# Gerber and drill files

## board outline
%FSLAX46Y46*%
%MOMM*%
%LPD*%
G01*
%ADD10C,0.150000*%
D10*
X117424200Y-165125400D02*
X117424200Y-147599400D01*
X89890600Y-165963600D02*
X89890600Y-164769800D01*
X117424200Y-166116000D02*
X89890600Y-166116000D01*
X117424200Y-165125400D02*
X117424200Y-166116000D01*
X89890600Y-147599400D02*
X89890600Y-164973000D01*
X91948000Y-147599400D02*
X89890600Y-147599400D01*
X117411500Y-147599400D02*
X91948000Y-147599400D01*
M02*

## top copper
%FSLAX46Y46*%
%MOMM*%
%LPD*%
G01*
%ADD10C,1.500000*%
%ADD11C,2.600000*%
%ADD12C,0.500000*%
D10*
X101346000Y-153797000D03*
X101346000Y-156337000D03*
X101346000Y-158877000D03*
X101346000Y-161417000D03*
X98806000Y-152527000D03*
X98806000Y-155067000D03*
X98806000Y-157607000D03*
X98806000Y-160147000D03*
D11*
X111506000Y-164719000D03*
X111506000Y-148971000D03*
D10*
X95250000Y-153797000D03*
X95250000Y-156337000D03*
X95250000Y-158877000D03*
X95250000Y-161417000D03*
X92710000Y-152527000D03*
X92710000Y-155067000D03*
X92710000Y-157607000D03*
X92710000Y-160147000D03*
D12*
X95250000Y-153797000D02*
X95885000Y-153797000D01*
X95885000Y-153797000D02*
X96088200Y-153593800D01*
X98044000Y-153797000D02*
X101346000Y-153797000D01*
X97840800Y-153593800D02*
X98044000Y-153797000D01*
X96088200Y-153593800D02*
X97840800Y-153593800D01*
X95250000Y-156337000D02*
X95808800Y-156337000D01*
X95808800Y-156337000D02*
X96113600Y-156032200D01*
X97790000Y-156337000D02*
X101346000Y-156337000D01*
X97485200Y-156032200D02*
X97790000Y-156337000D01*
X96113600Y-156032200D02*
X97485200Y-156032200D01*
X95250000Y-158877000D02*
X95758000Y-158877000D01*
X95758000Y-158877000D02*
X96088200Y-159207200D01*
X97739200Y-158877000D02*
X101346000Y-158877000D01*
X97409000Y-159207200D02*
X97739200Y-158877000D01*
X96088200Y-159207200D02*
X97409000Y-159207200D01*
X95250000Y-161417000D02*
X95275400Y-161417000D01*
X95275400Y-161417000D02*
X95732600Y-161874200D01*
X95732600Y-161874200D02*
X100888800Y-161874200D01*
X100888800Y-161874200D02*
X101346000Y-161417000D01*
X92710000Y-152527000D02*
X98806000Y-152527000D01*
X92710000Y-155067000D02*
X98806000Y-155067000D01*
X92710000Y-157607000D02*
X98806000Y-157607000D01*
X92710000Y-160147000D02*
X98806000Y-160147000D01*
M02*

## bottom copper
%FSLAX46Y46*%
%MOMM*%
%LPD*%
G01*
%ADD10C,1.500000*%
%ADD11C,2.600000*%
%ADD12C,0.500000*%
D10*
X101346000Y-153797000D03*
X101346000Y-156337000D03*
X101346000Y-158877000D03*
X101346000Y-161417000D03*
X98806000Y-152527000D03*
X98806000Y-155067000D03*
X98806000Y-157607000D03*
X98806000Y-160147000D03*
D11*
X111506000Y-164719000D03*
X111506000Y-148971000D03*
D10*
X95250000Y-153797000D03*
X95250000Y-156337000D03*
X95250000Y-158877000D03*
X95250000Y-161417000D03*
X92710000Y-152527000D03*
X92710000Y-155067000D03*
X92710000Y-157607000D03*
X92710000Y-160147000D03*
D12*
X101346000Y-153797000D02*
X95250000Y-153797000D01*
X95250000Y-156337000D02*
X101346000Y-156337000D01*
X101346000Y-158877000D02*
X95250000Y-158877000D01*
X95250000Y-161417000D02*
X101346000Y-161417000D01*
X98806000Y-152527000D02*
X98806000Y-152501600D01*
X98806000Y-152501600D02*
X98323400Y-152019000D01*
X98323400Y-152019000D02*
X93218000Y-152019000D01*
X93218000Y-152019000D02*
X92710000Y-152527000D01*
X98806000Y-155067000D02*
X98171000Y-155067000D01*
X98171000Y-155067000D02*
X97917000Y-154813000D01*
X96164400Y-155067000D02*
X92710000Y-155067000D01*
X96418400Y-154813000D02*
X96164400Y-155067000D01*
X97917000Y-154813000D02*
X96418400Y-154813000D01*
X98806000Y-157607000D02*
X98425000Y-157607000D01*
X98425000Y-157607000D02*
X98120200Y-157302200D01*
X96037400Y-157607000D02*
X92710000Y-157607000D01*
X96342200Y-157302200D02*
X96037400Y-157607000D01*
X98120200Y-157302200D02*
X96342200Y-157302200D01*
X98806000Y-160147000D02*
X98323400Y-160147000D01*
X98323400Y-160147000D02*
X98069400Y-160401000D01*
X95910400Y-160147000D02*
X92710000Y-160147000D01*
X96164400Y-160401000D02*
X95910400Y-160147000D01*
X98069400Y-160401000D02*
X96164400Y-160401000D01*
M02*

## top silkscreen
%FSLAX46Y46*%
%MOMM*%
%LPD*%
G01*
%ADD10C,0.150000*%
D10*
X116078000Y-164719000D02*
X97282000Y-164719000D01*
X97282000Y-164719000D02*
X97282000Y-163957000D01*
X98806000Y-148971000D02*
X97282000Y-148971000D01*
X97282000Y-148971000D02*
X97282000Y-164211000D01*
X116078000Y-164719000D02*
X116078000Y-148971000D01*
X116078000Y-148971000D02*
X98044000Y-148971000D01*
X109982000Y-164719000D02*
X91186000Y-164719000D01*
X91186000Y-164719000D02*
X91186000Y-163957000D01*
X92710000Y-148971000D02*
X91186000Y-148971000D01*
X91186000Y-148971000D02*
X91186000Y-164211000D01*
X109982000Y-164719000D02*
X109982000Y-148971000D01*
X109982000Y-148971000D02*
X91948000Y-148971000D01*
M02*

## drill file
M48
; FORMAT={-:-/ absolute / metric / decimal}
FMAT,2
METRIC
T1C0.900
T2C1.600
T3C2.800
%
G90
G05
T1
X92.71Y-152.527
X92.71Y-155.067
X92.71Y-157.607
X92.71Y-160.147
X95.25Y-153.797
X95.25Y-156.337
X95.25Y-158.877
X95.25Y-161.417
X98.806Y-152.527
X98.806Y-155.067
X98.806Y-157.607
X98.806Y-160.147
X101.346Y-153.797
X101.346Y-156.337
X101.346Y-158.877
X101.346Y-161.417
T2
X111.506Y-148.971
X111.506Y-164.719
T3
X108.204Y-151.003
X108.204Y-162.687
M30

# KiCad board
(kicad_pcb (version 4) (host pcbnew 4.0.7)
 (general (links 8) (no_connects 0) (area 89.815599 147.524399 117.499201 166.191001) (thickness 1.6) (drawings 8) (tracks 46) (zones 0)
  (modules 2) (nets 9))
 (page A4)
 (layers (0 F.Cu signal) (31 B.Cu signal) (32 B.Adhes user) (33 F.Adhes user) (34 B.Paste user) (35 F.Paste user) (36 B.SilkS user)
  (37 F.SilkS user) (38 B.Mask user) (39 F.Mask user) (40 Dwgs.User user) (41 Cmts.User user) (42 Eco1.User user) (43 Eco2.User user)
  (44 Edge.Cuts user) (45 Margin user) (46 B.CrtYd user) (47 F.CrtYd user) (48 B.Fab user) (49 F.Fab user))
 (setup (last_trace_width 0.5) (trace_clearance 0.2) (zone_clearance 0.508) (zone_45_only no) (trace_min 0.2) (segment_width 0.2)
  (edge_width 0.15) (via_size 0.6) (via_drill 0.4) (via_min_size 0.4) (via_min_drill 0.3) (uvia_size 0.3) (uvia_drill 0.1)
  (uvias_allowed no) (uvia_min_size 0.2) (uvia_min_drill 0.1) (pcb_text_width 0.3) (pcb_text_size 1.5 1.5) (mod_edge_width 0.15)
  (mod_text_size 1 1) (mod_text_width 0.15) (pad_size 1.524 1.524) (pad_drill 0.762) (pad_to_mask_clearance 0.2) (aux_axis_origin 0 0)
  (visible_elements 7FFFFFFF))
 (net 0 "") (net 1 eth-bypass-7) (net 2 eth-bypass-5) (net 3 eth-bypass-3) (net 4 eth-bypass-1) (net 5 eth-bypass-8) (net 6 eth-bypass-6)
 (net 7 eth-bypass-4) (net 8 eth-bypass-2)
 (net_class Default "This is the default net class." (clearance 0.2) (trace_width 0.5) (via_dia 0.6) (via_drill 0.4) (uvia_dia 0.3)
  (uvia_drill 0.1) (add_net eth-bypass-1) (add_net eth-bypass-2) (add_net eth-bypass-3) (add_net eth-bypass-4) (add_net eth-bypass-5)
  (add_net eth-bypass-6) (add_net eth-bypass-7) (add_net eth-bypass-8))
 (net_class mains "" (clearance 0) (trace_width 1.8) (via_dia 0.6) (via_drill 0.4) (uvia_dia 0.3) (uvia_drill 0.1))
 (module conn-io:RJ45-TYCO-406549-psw (layer F.Cu) (at 103.124 156.337 180)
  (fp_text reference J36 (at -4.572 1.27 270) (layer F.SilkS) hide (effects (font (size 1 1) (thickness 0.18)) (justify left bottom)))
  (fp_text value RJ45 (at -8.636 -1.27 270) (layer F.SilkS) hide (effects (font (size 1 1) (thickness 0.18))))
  (fp_line (start -12.954 -8.382) (end 5.842 -8.382) (layer F.SilkS) (width 0.15))
  (fp_line (start 5.842 -8.382) (end 5.842 -7.62) (layer F.SilkS) (width 0.15))
  (fp_line (start 4.318 7.366) (end 5.842 7.366) (layer F.SilkS) (width 0.15))
  (fp_line (start 5.842 7.366) (end 5.842 -7.874) (layer F.SilkS) (width 0.15))
  (fp_line (start -12.954 -8.382) (end -12.954 7.366) (layer F.SilkS) (width 0.15))
  (fp_line (start -12.954 7.366) (end 5.08 7.366) (layer F.SilkS) (width 0.15))
  (pad 7 thru_hole circle (at 1.778 2.54 180) (size 1.5 1.5) (drill 0.9) (layers *.Cu *.Mask) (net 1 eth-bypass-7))
  (pad 5 thru_hole circle (at 1.778 0 180) (size 1.5 1.5) (drill 0.9) (layers *.Cu *.Mask) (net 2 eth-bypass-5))
  (pad 3 thru_hole circle (at 1.778 -2.54 180) (size 1.5 1.5) (drill 0.9) (layers *.Cu *.Mask) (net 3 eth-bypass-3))
  (pad 1 thru_hole circle (at 1.778 -5.08 180) (size 1.5 1.5) (drill 0.9) (layers *.Cu *.Mask) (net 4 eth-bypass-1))
  (pad 8 thru_hole circle (at 4.318 3.81 180) (size 1.5 1.5) (drill 0.9) (layers *.Cu *.Mask) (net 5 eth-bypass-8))
  (pad 6 thru_hole circle (at 4.318 1.27 180) (size 1.5 1.5) (drill 0.9) (layers *.Cu *.Mask) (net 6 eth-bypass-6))
  (pad 4 thru_hole circle (at 4.318 -1.27 180) (size 1.5 1.5) (drill 0.9) (layers *.Cu *.Mask) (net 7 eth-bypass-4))
  (pad 2 thru_hole circle (at 4.318 -3.81 180) (size 1.5 1.5) (drill 0.9) (layers *.Cu *.Mask) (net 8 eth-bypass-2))
  (pad SH thru_hole circle (at -8.382 -8.382 180) (size 2.6 2.6) (drill 1.6) (layers *.Cu *.Mask))
  (pad SH thru_hole circle (at -8.382 7.366 180) (size 2.6 2.6) (drill 1.6) (layers *.Cu *.Mask))
  (pad "" np_thru_hole circle (at -5.08 -6.35 180) (size 2.8 2.8) (drill 2.8) (layers *.Cu))
  (pad "" np_thru_hole circle (at -5.08 5.334 180) (size 2.8 2.8) (drill 2.8) (layers *.Cu)))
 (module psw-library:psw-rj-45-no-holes (layer F.Cu) (at 97.028 156.337 180)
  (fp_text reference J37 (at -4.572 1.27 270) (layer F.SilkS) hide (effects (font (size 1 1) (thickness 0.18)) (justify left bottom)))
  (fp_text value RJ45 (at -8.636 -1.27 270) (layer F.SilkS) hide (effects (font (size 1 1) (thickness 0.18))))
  (fp_line (start -12.954 -8.382) (end 5.842 -8.382) (layer F.SilkS) (width 0.15))
  (fp_line (start 5.842 -8.382) (end 5.842 -7.62) (layer F.SilkS) (width 0.15))
  (fp_line (start 4.318 7.366) (end 5.842 7.366) (layer F.SilkS) (width 0.15))
  (fp_line (start 5.842 7.366) (end 5.842 -7.874) (layer F.SilkS) (width 0.15))
  (fp_line (start -12.954 -8.382) (end -12.954 7.366) (layer F.SilkS) (width 0.15))
  (fp_line (start -12.954 7.366) (end 5.08 7.366) (layer F.SilkS) (width 0.15))
  (pad 7 thru_hole circle (at 1.778 2.54 180) (size 1.5 1.5) (drill 0.9) (layers *.Cu *.Mask) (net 1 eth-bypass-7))
  (pad 5 thru_hole circle (at 1.778 0 180) (size 1.5 1.5) (drill 0.9) (layers *.Cu *.Mask) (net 2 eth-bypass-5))
  (pad 3 thru_hole circle (at 1.778 -2.54 180) (size 1.5 1.5) (drill 0.9) (layers *.Cu *.Mask) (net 3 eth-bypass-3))
  (pad 1 thru_hole circle (at 1.778 -5.08 180) (size 1.5 1.5) (drill 0.9) (layers *.Cu *.Mask) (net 4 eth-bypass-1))
  (pad 8 thru_hole circle (at 4.318 3.81 180) (size 1.5 1.5) (drill 0.9) (layers *.Cu *.Mask) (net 5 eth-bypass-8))
  (pad 6 thru_hole circle (at 4.318 1.27 180) (size 1.5 1.5) (drill 0.9) (layers *.Cu *.Mask) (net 6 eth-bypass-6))
  (pad 4 thru_hole circle (at 4.318 -1.27 180) (size 1.5 1.5) (drill 0.9) (layers *.Cu *.Mask) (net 7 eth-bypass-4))
  (pad 2 thru_hole circle (at 4.318 -3.81 180) (size 1.5 1.5) (drill 0.9) (layers *.Cu *.Mask) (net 8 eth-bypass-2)))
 (gr_line (start 117.4242 165.1254) (end 117.4242 147.5994) (angle 90) (layer Edge.Cuts) (width 0.15))
 (gr_line (start 89.8906 165.9636) (end 89.8906 164.7698) (angle 90) (layer Edge.Cuts) (width 0.15))
 (gr_line (start 117.4242 166.116) (end 89.8906 166.116) (angle 90) (layer Edge.Cuts) (width 0.15))
 (gr_line (start 117.4242 165.1254) (end 117.4242 166.116) (angle 90) (layer Edge.Cuts) (width 0.15))
 (gr_line (start 89.8906 147.5994) (end 89.8906 164.973) (angle 90) (layer Edge.Cuts) (width 0.15))
 (gr_line (start 91.948 147.5994) (end 89.8906 147.5994) (angle 90) (layer Edge.Cuts) (width 0.15))
 (gr_line (start 117.4115 147.5994) (end 91.948 147.5994) (angle 90) (layer Edge.Cuts) (width 0.15))
 (segment (start 95.25 153.797) (end 95.885 153.797) (width 0.5) (layer F.Cu) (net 1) (status C00000))
 (segment (start 95.885 153.797) (end 96.0882 153.5938) (width 0.5) (layer F.Cu) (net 1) (status 400000))
 (segment (start 98.044 153.797) (end 101.346 153.797) (width 0.5) (layer F.Cu) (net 1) (status 800000))
 (segment (start 97.8408 153.5938) (end 98.044 153.797) (width 0.5) (layer F.Cu) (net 1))
 (segment (start 96.0882 153.5938) (end 97.8408 153.5938) (width 0.5) (layer F.Cu) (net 1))
 (segment (start 101.346 153.797) (end 95.25 153.797) (width 0.5) (layer B.Cu) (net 1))
 (segment (start 95.25 156.337) (end 95.8088 156.337) (width 0.5) (layer F.Cu) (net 2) (status C00000))
 (segment (start 95.8088 156.337) (end 96.1136 156.0322) (width 0.5) (layer F.Cu) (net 2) (status 400000))
 (segment (start 97.79 156.337) (end 101.346 156.337) (width 0.5) (layer F.Cu) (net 2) (status 800000))
 (segment (start 97.4852 156.0322) (end 97.79 156.337) (width 0.5) (layer F.Cu) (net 2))
 (segment (start 96.1136 156.0322) (end 97.4852 156.0322) (width 0.5) (layer F.Cu) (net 2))
 (segment (start 95.25 156.337) (end 101.346 156.337) (width 0.5) (layer B.Cu) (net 2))
 (segment (start 95.25 158.877) (end 95.758 158.877) (width 0.5) (layer F.Cu) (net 3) (status C00000))
 (segment (start 95.758 158.877) (end 96.0882 159.2072) (width 0.5) (layer F.Cu) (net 3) (status 400000))
 (segment (start 97.7392 158.877) (end 101.346 158.877) (width 0.5) (layer F.Cu) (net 3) (status 800000))
 (segment (start 97.409 159.2072) (end 97.7392 158.877) (width 0.5) (layer F.Cu) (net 3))
 (segment (start 96.0882 159.2072) (end 97.409 159.2072) (width 0.5) (layer F.Cu) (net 3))
 (segment (start 101.346 158.877) (end 95.25 158.877) (width 0.5) (layer B.Cu) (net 3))
 (segment (start 95.25 161.417) (end 95.2754 161.417) (width 0.5) (layer F.Cu) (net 4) (status C00000))
 (segment (start 95.2754 161.417) (end 95.7326 161.8742) (width 0.5) (layer F.Cu) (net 4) (status C00000))
 (segment (start 95.7326 161.8742) (end 100.8888 161.8742) (width 0.5) (layer F.Cu) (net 4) (status C00000))
 (segment (start 100.8888 161.8742) (end 101.346 161.417) (width 0.5) (layer F.Cu) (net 4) (status C00000))
 (segment (start 95.25 161.417) (end 101.346 161.417) (width 0.5) (layer B.Cu) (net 4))
 (segment (start 98.806 152.527) (end 98.806 152.5016) (width 0.5) (layer B.Cu) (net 5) (status C00000))
 (segment (start 98.806 152.5016) (end 98.3234 152.019) (width 0.5) (layer B.Cu) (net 5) (status C00000))
 (segment (start 98.3234 152.019) (end 93.218 152.019) (width 0.5) (layer B.Cu) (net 5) (status C00000))
 (segment (start 93.218 152.019) (end 92.71 152.527) (width 0.5) (layer B.Cu) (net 5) (status C00000))
 (segment (start 92.71 152.527) (end 98.806 152.527) (width 0.5) (layer F.Cu) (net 5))
 (segment (start 98.806 155.067) (end 98.171 155.067) (width 0.5) (layer B.Cu) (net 6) (status C00000))
 (segment (start 98.171 155.067) (end 97.917 154.813) (width 0.5) (layer B.Cu) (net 6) (status 400000))
 (segment (start 96.1644 155.067) (end 92.71 155.067) (width 0.5) (layer B.Cu) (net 6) (status 800000))
 (segment (start 96.4184 154.813) (end 96.1644 155.067) (width 0.5) (layer B.Cu) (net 6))
 (segment (start 97.917 154.813) (end 96.4184 154.813) (width 0.5) (layer B.Cu) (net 6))
 (segment (start 92.71 155.067) (end 98.806 155.067) (width 0.5) (layer F.Cu) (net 6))
 (segment (start 98.806 157.607) (end 98.425 157.607) (width 0.5) (layer B.Cu) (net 7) (status C00000))
 (segment (start 98.425 157.607) (end 98.1202 157.3022) (width 0.5) (layer B.Cu) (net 7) (status 400000))
 (segment (start 96.0374 157.607) (end 92.71 157.607) (width 0.5) (layer B.Cu) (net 7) (status 800000))
 (segment (start 96.3422 157.3022) (end 96.0374 157.607) (width 0.5) (layer B.Cu) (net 7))
 (segment (start 98.1202 157.3022) (end 96.3422 157.3022) (width 0.5) (layer B.Cu) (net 7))
 (segment (start 92.71 157.607) (end 98.806 157.607) (width 0.5) (layer F.Cu) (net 7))
 (segment (start 98.806 160.147) (end 98.3234 160.147) (width 0.5) (layer B.Cu) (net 8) (status C00000))
 (segment (start 98.3234 160.147) (end 98.0694 160.401) (width 0.5) (layer B.Cu) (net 8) (status 400000))
 (segment (start 95.9104 160.147) (end 92.71 160.147) (width 0.5) (layer B.Cu) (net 8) (status 800000))
 (segment (start 96.1644 160.401) (end 95.9104 160.147) (width 0.5) (layer B.Cu) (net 8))
 (segment (start 98.0694 160.401) (end 96.1644 160.401) (width 0.5) (layer B.Cu) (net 8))
 (segment (start 92.71 160.147) (end 98.806 160.147) (width 0.5) (layer F.Cu) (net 8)))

